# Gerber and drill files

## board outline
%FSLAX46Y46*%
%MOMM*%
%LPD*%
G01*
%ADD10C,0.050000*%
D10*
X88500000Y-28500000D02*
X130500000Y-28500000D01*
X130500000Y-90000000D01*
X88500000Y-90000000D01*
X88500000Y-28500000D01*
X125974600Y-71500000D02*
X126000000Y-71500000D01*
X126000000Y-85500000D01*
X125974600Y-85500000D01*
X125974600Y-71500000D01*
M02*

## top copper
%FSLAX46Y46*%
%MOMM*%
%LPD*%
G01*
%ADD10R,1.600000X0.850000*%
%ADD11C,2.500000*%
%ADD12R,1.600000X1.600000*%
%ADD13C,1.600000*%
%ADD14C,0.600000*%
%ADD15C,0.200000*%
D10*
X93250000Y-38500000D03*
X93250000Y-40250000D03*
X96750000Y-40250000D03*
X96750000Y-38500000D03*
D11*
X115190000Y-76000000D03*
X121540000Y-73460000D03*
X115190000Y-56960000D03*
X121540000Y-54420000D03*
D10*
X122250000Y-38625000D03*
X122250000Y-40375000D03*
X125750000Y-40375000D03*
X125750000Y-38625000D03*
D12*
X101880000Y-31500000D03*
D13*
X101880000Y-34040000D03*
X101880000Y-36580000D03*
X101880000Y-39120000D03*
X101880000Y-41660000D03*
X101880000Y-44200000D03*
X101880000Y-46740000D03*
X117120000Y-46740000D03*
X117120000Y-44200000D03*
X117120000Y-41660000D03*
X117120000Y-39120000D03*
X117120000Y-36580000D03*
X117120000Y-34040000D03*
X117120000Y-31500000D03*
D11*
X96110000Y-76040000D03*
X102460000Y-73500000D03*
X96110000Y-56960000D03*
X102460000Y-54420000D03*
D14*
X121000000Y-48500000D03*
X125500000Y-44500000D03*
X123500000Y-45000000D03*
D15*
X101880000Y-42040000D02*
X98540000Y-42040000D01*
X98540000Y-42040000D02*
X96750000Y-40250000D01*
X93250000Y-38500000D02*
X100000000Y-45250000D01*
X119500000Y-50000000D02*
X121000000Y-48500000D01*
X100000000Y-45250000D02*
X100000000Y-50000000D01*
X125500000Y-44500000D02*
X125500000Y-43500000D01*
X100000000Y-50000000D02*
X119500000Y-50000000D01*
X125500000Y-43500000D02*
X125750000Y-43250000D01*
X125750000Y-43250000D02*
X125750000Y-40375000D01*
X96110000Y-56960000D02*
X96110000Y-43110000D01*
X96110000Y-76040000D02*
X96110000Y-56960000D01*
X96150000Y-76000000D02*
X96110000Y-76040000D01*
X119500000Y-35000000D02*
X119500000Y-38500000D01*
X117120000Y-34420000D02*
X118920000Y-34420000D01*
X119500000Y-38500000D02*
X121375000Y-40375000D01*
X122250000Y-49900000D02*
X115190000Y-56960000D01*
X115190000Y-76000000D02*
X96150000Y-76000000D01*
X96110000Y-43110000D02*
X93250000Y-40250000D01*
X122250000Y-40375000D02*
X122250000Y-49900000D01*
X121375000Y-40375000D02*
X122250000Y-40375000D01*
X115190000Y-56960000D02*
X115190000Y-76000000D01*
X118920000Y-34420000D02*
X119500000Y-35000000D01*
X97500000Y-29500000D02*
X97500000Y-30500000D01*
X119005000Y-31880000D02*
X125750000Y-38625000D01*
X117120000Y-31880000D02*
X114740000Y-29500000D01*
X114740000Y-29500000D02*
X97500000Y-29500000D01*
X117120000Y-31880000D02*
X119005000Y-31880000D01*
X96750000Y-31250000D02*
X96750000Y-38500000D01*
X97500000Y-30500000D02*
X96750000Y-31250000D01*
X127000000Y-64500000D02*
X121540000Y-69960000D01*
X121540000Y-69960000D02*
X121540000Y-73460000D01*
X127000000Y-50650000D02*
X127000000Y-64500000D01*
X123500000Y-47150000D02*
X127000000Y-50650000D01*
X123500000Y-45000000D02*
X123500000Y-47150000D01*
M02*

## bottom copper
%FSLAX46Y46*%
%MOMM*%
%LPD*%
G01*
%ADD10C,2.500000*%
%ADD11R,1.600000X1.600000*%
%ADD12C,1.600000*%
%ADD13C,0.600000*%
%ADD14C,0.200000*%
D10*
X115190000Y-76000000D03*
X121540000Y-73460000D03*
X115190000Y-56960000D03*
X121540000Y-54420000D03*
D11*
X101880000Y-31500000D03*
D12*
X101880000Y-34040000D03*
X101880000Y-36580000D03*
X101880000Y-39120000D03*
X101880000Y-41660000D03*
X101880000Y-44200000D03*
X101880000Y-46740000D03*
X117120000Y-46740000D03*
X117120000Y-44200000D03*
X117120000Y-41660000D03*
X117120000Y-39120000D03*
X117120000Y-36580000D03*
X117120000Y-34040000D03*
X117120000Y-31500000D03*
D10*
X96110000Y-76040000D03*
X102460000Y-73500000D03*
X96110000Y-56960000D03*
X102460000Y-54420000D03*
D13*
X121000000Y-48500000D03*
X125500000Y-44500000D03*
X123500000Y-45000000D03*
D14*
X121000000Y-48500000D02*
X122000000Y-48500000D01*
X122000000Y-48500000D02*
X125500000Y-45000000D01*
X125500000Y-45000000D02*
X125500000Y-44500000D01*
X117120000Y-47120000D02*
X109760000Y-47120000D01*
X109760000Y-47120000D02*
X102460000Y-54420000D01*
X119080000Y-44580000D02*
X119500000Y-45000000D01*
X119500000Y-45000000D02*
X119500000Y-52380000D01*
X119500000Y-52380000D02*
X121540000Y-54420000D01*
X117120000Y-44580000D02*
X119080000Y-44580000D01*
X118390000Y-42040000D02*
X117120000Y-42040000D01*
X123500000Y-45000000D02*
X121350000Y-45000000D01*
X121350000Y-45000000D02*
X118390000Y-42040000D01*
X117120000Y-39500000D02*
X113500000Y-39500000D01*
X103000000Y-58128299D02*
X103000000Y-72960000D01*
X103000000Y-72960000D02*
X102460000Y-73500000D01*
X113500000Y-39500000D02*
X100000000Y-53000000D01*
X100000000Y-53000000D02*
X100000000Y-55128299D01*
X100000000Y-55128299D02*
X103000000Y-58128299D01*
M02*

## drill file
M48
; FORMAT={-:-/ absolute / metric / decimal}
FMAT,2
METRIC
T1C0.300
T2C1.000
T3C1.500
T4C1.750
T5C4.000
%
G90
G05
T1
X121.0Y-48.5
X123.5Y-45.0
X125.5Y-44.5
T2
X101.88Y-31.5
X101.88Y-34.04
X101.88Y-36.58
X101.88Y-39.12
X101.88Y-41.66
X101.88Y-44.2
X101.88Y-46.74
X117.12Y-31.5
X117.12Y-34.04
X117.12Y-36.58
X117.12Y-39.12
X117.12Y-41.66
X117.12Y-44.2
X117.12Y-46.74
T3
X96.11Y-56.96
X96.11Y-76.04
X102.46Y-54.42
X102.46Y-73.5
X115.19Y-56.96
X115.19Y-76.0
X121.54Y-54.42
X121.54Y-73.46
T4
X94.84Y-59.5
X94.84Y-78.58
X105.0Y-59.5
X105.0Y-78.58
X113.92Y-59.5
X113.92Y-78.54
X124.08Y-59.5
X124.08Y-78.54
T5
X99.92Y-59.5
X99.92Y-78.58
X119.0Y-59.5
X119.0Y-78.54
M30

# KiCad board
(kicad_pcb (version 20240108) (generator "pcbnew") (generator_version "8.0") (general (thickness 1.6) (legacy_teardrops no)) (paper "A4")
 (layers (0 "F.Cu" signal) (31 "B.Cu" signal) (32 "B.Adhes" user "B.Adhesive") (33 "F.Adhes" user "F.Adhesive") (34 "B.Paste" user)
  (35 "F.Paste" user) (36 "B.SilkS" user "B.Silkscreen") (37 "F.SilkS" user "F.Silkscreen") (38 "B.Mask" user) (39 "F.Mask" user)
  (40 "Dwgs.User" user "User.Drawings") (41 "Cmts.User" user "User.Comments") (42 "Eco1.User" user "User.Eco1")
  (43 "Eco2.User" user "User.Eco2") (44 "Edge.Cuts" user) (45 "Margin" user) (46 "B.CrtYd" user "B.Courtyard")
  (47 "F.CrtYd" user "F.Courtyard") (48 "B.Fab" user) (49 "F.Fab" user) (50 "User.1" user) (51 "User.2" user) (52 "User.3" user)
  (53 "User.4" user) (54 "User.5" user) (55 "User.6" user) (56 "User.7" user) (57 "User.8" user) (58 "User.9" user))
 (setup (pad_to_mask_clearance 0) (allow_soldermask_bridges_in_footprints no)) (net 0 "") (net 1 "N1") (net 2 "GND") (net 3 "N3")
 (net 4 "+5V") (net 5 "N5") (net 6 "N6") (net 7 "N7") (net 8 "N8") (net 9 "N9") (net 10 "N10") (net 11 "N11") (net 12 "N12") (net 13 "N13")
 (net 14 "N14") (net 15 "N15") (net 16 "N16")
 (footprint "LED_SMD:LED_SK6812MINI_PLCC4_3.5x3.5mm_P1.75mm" (layer "F.Cu") (at 95 39.375)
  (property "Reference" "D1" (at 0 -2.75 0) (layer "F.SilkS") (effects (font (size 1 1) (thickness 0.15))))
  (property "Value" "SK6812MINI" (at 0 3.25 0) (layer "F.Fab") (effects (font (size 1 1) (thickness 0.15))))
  (pad "1" smd rect (at -1.75 -0.875) (size 1.6 0.85) (layers "F.Cu" "F.Paste" "F.Mask") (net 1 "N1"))
  (pad "2" smd rect (at -1.75 0.875) (size 1.6 0.85) (layers "F.Cu" "F.Paste" "F.Mask") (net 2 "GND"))
  (pad "3" smd rect (at 1.75 0.875) (size 1.6 0.85) (layers "F.Cu" "F.Paste" "F.Mask") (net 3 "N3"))
  (pad "4" smd rect (at 1.75 -0.875) (size 1.6 0.85) (layers "F.Cu" "F.Paste" "F.Mask") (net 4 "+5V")))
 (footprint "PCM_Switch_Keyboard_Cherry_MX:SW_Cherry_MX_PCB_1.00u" (layer "F.Cu") (at 119 78.54)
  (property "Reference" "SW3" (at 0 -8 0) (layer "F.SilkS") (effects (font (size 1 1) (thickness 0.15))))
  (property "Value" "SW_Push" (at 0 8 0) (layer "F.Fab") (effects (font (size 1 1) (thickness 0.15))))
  (pad "" np_thru_hole circle (at -5.08 0) (size 1.75 1.75) (drill 1.75) (layers "*.Cu" "*.Mask"))
  (pad "" np_thru_hole circle (at 0 0) (size 4 4) (drill 4) (layers "*.Cu" "*.Mask"))
  (pad "" np_thru_hole circle (at 5.08 0) (size 1.75 1.75) (drill 1.75) (layers "*.Cu" "*.Mask"))
  (pad "1" thru_hole circle (at -3.81 -2.54) (size 2.5 2.5) (drill 1.5) (layers "*.Cu" "*.Mask") (remove_unused_layers no) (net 2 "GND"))
  (pad "2" thru_hole circle (at 2.54 -5.08) (size 2.5 2.5) (drill 1.5) (layers "*.Cu" "*.Mask") (remove_unused_layers no) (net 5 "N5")))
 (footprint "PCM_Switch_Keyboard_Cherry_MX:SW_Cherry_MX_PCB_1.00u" (layer "F.Cu") (at 119 59.5)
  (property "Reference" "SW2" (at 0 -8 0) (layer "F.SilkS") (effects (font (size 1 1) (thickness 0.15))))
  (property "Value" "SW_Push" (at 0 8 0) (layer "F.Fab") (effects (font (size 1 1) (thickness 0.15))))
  (pad "" np_thru_hole circle (at -5.08 0) (size 1.75 1.75) (drill 1.75) (layers "*.Cu" "*.Mask"))
  (pad "" np_thru_hole circle (at 0 0) (size 4 4) (drill 4) (layers "*.Cu" "*.Mask"))
  (pad "" np_thru_hole circle (at 5.08 0) (size 1.75 1.75) (drill 1.75) (layers "*.Cu" "*.Mask"))
  (pad "1" thru_hole circle (at -3.81 -2.54) (size 2.5 2.5) (drill 1.5) (layers "*.Cu" "*.Mask") (remove_unused_layers no) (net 2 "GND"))
  (pad "2" thru_hole circle (at 2.54 -5.08) (size 2.5 2.5) (drill 1.5) (layers "*.Cu" "*.Mask") (remove_unused_layers no) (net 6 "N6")))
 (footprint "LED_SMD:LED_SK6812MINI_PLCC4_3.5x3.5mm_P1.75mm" (layer "F.Cu") (at 124 39.5)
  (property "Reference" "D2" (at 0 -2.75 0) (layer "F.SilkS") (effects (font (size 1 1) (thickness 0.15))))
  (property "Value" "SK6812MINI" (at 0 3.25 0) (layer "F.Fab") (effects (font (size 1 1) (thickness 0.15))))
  (pad "1" smd rect (at -1.75 -0.875) (size 1.6 0.85) (layers "F.Cu" "F.Paste" "F.Mask") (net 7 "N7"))
  (pad "2" smd rect (at -1.75 0.875) (size 1.6 0.85) (layers "F.Cu" "F.Paste" "F.Mask") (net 2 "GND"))
  (pad "3" smd rect (at 1.75 0.875) (size 1.6 0.85) (layers "F.Cu" "F.Paste" "F.Mask") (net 1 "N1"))
  (pad "4" smd rect (at 1.75 -0.875) (size 1.6 0.85) (layers "F.Cu" "F.Paste" "F.Mask") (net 4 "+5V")))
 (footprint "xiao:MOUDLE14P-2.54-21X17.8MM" (layer "F.Cu") (at 109.5 39.12 90)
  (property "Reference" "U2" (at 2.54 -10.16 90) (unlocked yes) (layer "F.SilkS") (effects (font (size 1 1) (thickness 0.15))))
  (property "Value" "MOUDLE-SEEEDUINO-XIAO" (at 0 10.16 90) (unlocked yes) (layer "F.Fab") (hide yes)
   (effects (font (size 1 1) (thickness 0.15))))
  (pad "1" thru_hole rect (at 7.62 -7.62 90) (size 1.6 1.6) (drill 1) (layers "*.Cu" "*.Mask") (remove_unused_layers no) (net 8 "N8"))
  (pad "2" thru_hole circle (at 5.08 -7.62 90) (size 1.6 1.6) (drill 1) (layers "*.Cu" "*.Mask") (remove_unused_layers no) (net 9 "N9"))
  (pad "3" thru_hole circle (at 2.54 -7.62 90) (size 1.6 1.6) (drill 1) (layers "*.Cu" "*.Mask") (remove_unused_layers no) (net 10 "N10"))
  (pad "4" thru_hole circle (at 0 -7.62 90) (size 1.6 1.6) (drill 1) (layers "*.Cu" "*.Mask") (remove_unused_layers no) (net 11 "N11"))
  (pad "5" thru_hole circle (at -2.54 -7.62 90) (size 1.6 1.6) (drill 1) (layers "*.Cu" "*.Mask") (remove_unused_layers no) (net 3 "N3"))
  (pad "6" thru_hole circle (at -5.08 -7.62 90) (size 1.6 1.6) (drill 1) (layers "*.Cu" "*.Mask") (remove_unused_layers no) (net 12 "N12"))
  (pad "7" thru_hole circle (at -7.62 -7.62 90) (size 1.6 1.6) (drill 1) (layers "*.Cu" "*.Mask") (remove_unused_layers no) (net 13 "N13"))
  (pad "8" thru_hole circle (at -7.62 7.62 90) (size 1.6 1.6) (drill 1) (layers "*.Cu" "*.Mask") (remove_unused_layers no) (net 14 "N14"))
  (pad "9" thru_hole circle (at -5.08 7.62 90) (size 1.6 1.6) (drill 1) (layers "*.Cu" "*.Mask") (remove_unused_layers no) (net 6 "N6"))
  (pad "10" thru_hole circle (at -2.54 7.62 90) (size 1.6 1.6) (drill 1) (layers "*.Cu" "*.Mask") (remove_unused_layers no) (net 5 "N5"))
  (pad "11" thru_hole circle (at 0 7.62 90) (size 1.6 1.6) (drill 1) (layers "*.Cu" "*.Mask") (remove_unused_layers no) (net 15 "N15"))
  (pad "12" thru_hole circle (at 2.54 7.62 90) (size 1.6 1.6) (drill 1) (layers "*.Cu" "*.Mask") (remove_unused_layers no) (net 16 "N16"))
  (pad "13" thru_hole circle (at 5.08 7.62 90) (size 1.6 1.6) (drill 1) (layers "*.Cu" "*.Mask") (remove_unused_layers no) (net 2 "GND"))
  (pad "14" thru_hole circle (at 7.62 7.62 90) (size 1.6 1.6) (drill 1) (layers "*.Cu" "*.Mask") (remove_unused_layers no) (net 4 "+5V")))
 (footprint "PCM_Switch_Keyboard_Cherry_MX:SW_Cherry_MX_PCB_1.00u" (layer "F.Cu") (at 99.92 78.58)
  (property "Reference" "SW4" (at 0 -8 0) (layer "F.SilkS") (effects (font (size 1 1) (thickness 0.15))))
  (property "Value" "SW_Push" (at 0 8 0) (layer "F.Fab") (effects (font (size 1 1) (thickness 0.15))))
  (pad "" np_thru_hole circle (at -5.08 0) (size 1.75 1.75) (drill 1.75) (layers "*.Cu" "*.Mask"))
  (pad "" np_thru_hole circle (at 0 0) (size 4 4) (drill 4) (layers "*.Cu" "*.Mask"))
  (pad "" np_thru_hole circle (at 5.08 0) (size 1.75 1.75) (drill 1.75) (layers "*.Cu" "*.Mask"))
  (pad "1" thru_hole circle (at -3.81 -2.54) (size 2.5 2.5) (drill 1.5) (layers "*.Cu" "*.Mask") (remove_unused_layers no) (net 2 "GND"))
  (pad "2" thru_hole circle (at 2.54 -5.08) (size 2.5 2.5) (drill 1.5) (layers "*.Cu" "*.Mask") (remove_unused_layers no) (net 15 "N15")))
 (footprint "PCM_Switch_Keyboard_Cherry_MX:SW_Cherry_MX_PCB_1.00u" (layer "F.Cu") (at 99.92 59.5)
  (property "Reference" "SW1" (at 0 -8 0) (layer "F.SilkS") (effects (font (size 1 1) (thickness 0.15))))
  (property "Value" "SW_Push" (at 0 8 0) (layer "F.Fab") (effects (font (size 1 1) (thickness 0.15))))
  (pad "" np_thru_hole circle (at -5.08 0) (size 1.75 1.75) (drill 1.75) (layers "*.Cu" "*.Mask"))
  (pad "" np_thru_hole circle (at 0 0) (size 4 4) (drill 4) (layers "*.Cu" "*.Mask"))
  (pad "" np_thru_hole circle (at 5.08 0) (size 1.75 1.75) (drill 1.75) (layers "*.Cu" "*.Mask"))
  (pad "1" thru_hole circle (at -3.81 -2.54) (size 2.5 2.5) (drill 1.5) (layers "*.Cu" "*.Mask") (remove_unused_layers no) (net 2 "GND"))
  (pad "2" thru_hole circle (at 2.54 -5.08) (size 2.5 2.5) (drill 1.5) (layers "*.Cu" "*.Mask") (remove_unused_layers no) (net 14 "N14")))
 (gr_rect (start 88.5 28.5) (end 130.5 90) (stroke (width 0.05) (type default)) (fill none) (layer "Edge.Cuts"))
 (gr_rect (start 125.9746 71.5) (end 126 85.5) (stroke (width 0.05) (type default)) (fill none) (layer "Edge.Cuts"))
 (segment (start 101.88 42.04) (end 98.54 42.04) (width 0.2) (layer "F.Cu") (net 3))
 (segment (start 98.54 42.04) (end 96.75 40.25) (width 0.2) (layer "F.Cu") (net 3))
 (segment (start 93.25 38.5) (end 100 45.25) (width 0.2) (layer "F.Cu") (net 1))
 (segment (start 119.5 50) (end 121 48.5) (width 0.2) (layer "F.Cu") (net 1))
 (segment (start 100 45.25) (end 100 50) (width 0.2) (layer "F.Cu") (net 1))
 (segment (start 125.5 44.5) (end 125.5 43.5) (width 0.2) (layer "F.Cu") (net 1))
 (segment (start 100 50) (end 119.5 50) (width 0.2) (layer "F.Cu") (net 1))
 (segment (start 125.5 43.5) (end 125.75 43.25) (width 0.2) (layer "F.Cu") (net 1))
 (segment (start 125.75 43.25) (end 125.75 40.375) (width 0.2) (layer "F.Cu") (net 1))
 (via (at 121 48.5) (size 0.6) (drill 0.3) (layers "F.Cu" "B.Cu") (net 1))
 (via (at 125.5 44.5) (size 0.6) (drill 0.3) (layers "F.Cu" "B.Cu") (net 1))
 (segment (start 121 48.5) (end 122 48.5) (width 0.2) (layer "B.Cu") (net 1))
 (segment (start 122 48.5) (end 125.5 45) (width 0.2) (layer "B.Cu") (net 1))
 (segment (start 125.5 45) (end 125.5 44.5) (width 0.2) (layer "B.Cu") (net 1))
 (segment (start 96.11 56.96) (end 96.11 43.11) (width 0.2) (layer "F.Cu") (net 2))
 (segment (start 96.11 76.04) (end 96.11 56.96) (width 0.2) (layer "F.Cu") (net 2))
 (segment (start 96.15 76) (end 96.11 76.04) (width 0.2) (layer "F.Cu") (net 2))
 (segment (start 119.5 35) (end 119.5 38.5) (width 0.2) (layer "F.Cu") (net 2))
 (segment (start 117.12 34.42) (end 118.92 34.42) (width 0.2) (layer "F.Cu") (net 2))
 (segment (start 119.5 38.5) (end 121.375 40.375) (width 0.2) (layer "F.Cu") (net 2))
 (segment (start 122.25 49.9) (end 115.19 56.96) (width 0.2) (layer "F.Cu") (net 2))
 (segment (start 115.19 76) (end 96.15 76) (width 0.2) (layer "F.Cu") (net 2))
 (segment (start 96.11 43.11) (end 93.25 40.25) (width 0.2) (layer "F.Cu") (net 2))
 (segment (start 122.25 40.375) (end 122.25 49.9) (width 0.2) (layer "F.Cu") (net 2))
 (segment (start 121.375 40.375) (end 122.25 40.375) (width 0.2) (layer "F.Cu") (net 2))
 (segment (start 115.19 56.96) (end 115.19 76) (width 0.2) (layer "F.Cu") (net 2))
 (segment (start 118.92 34.42) (end 119.5 35) (width 0.2) (layer "F.Cu") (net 2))
 (segment (start 97.5 29.5) (end 97.5 30.5) (width 0.2) (layer "F.Cu") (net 4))
 (segment (start 119.005 31.88) (end 125.75 38.625) (width 0.2) (layer "F.Cu") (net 4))
 (segment (start 117.12 31.88) (end 114.74 29.5) (width 0.2) (layer "F.Cu") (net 4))
 (segment (start 114.74 29.5) (end 97.5 29.5) (width 0.2) (layer "F.Cu") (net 4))
 (segment (start 117.12 31.88) (end 119.005 31.88) (width 0.2) (layer "F.Cu") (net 4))
 (segment (start 96.75 31.25) (end 96.75 38.5) (width 0.2) (layer "F.Cu") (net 4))
 (segment (start 97.5 30.5) (end 96.75 31.25) (width 0.2) (layer "F.Cu") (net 4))
 (segment (start 117.12 47.12) (end 109.76 47.12) (width 0.2) (layer "B.Cu") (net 14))
 (segment (start 109.76 47.12) (end 102.46 54.42) (width 0.2) (layer "B.Cu") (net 14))
 (segment (start 119.08 44.58) (end 119.5 45) (width 0.2) (layer "B.Cu") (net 6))
 (segment (start 119.5 45) (end 119.5 52.38) (width 0.2) (layer "B.Cu") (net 6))
 (segment (start 119.5 52.38) (end 121.54 54.42) (width 0.2) (layer "B.Cu") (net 6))
 (segment (start 117.12 44.58) (end 119.08 44.58) (width 0.2) (layer "B.Cu") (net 6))
 (segment (start 127 64.5) (end 121.54 69.96) (width 0.2) (layer "F.Cu") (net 5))
 (segment (start 121.54 69.96) (end 121.54 73.46) (width 0.2) (layer "F.Cu") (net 5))
 (segment (start 127 50.65) (end 127 64.5) (width 0.2) (layer "F.Cu") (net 5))
 (segment (start 123.5 47.15) (end 127 50.65) (width 0.2) (layer "F.Cu") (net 5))
 (segment (start 123.5 45) (end 123.5 47.15) (width 0.2) (layer "F.Cu") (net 5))
 (via (at 123.5 45) (size 0.6) (drill 0.3) (layers "F.Cu" "B.Cu") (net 5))
 (segment (start 118.39 42.04) (end 117.12 42.04) (width 0.2) (layer "B.Cu") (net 5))
 (segment (start 123.5 45) (end 121.35 45) (width 0.2) (layer "B.Cu") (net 5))
 (segment (start 121.35 45) (end 118.39 42.04) (width 0.2) (layer "B.Cu") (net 5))
 (segment (start 117.12 39.5) (end 113.5 39.5) (width 0.2) (layer "B.Cu") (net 15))
 (segment (start 103 58.128299) (end 103 72.96) (width 0.2) (layer "B.Cu") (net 15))
 (segment (start 103 72.96) (end 102.46 73.5) (width 0.2) (layer "B.Cu") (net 15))
 (segment (start 113.5 39.5) (end 100 53) (width 0.2) (layer "B.Cu") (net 15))
 (segment (start 100 53) (end 100 55.128299) (width 0.2) (layer "B.Cu") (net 15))
 (segment (start 100 55.128299) (end 103 58.128299) (width 0.2) (layer "B.Cu") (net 15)))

